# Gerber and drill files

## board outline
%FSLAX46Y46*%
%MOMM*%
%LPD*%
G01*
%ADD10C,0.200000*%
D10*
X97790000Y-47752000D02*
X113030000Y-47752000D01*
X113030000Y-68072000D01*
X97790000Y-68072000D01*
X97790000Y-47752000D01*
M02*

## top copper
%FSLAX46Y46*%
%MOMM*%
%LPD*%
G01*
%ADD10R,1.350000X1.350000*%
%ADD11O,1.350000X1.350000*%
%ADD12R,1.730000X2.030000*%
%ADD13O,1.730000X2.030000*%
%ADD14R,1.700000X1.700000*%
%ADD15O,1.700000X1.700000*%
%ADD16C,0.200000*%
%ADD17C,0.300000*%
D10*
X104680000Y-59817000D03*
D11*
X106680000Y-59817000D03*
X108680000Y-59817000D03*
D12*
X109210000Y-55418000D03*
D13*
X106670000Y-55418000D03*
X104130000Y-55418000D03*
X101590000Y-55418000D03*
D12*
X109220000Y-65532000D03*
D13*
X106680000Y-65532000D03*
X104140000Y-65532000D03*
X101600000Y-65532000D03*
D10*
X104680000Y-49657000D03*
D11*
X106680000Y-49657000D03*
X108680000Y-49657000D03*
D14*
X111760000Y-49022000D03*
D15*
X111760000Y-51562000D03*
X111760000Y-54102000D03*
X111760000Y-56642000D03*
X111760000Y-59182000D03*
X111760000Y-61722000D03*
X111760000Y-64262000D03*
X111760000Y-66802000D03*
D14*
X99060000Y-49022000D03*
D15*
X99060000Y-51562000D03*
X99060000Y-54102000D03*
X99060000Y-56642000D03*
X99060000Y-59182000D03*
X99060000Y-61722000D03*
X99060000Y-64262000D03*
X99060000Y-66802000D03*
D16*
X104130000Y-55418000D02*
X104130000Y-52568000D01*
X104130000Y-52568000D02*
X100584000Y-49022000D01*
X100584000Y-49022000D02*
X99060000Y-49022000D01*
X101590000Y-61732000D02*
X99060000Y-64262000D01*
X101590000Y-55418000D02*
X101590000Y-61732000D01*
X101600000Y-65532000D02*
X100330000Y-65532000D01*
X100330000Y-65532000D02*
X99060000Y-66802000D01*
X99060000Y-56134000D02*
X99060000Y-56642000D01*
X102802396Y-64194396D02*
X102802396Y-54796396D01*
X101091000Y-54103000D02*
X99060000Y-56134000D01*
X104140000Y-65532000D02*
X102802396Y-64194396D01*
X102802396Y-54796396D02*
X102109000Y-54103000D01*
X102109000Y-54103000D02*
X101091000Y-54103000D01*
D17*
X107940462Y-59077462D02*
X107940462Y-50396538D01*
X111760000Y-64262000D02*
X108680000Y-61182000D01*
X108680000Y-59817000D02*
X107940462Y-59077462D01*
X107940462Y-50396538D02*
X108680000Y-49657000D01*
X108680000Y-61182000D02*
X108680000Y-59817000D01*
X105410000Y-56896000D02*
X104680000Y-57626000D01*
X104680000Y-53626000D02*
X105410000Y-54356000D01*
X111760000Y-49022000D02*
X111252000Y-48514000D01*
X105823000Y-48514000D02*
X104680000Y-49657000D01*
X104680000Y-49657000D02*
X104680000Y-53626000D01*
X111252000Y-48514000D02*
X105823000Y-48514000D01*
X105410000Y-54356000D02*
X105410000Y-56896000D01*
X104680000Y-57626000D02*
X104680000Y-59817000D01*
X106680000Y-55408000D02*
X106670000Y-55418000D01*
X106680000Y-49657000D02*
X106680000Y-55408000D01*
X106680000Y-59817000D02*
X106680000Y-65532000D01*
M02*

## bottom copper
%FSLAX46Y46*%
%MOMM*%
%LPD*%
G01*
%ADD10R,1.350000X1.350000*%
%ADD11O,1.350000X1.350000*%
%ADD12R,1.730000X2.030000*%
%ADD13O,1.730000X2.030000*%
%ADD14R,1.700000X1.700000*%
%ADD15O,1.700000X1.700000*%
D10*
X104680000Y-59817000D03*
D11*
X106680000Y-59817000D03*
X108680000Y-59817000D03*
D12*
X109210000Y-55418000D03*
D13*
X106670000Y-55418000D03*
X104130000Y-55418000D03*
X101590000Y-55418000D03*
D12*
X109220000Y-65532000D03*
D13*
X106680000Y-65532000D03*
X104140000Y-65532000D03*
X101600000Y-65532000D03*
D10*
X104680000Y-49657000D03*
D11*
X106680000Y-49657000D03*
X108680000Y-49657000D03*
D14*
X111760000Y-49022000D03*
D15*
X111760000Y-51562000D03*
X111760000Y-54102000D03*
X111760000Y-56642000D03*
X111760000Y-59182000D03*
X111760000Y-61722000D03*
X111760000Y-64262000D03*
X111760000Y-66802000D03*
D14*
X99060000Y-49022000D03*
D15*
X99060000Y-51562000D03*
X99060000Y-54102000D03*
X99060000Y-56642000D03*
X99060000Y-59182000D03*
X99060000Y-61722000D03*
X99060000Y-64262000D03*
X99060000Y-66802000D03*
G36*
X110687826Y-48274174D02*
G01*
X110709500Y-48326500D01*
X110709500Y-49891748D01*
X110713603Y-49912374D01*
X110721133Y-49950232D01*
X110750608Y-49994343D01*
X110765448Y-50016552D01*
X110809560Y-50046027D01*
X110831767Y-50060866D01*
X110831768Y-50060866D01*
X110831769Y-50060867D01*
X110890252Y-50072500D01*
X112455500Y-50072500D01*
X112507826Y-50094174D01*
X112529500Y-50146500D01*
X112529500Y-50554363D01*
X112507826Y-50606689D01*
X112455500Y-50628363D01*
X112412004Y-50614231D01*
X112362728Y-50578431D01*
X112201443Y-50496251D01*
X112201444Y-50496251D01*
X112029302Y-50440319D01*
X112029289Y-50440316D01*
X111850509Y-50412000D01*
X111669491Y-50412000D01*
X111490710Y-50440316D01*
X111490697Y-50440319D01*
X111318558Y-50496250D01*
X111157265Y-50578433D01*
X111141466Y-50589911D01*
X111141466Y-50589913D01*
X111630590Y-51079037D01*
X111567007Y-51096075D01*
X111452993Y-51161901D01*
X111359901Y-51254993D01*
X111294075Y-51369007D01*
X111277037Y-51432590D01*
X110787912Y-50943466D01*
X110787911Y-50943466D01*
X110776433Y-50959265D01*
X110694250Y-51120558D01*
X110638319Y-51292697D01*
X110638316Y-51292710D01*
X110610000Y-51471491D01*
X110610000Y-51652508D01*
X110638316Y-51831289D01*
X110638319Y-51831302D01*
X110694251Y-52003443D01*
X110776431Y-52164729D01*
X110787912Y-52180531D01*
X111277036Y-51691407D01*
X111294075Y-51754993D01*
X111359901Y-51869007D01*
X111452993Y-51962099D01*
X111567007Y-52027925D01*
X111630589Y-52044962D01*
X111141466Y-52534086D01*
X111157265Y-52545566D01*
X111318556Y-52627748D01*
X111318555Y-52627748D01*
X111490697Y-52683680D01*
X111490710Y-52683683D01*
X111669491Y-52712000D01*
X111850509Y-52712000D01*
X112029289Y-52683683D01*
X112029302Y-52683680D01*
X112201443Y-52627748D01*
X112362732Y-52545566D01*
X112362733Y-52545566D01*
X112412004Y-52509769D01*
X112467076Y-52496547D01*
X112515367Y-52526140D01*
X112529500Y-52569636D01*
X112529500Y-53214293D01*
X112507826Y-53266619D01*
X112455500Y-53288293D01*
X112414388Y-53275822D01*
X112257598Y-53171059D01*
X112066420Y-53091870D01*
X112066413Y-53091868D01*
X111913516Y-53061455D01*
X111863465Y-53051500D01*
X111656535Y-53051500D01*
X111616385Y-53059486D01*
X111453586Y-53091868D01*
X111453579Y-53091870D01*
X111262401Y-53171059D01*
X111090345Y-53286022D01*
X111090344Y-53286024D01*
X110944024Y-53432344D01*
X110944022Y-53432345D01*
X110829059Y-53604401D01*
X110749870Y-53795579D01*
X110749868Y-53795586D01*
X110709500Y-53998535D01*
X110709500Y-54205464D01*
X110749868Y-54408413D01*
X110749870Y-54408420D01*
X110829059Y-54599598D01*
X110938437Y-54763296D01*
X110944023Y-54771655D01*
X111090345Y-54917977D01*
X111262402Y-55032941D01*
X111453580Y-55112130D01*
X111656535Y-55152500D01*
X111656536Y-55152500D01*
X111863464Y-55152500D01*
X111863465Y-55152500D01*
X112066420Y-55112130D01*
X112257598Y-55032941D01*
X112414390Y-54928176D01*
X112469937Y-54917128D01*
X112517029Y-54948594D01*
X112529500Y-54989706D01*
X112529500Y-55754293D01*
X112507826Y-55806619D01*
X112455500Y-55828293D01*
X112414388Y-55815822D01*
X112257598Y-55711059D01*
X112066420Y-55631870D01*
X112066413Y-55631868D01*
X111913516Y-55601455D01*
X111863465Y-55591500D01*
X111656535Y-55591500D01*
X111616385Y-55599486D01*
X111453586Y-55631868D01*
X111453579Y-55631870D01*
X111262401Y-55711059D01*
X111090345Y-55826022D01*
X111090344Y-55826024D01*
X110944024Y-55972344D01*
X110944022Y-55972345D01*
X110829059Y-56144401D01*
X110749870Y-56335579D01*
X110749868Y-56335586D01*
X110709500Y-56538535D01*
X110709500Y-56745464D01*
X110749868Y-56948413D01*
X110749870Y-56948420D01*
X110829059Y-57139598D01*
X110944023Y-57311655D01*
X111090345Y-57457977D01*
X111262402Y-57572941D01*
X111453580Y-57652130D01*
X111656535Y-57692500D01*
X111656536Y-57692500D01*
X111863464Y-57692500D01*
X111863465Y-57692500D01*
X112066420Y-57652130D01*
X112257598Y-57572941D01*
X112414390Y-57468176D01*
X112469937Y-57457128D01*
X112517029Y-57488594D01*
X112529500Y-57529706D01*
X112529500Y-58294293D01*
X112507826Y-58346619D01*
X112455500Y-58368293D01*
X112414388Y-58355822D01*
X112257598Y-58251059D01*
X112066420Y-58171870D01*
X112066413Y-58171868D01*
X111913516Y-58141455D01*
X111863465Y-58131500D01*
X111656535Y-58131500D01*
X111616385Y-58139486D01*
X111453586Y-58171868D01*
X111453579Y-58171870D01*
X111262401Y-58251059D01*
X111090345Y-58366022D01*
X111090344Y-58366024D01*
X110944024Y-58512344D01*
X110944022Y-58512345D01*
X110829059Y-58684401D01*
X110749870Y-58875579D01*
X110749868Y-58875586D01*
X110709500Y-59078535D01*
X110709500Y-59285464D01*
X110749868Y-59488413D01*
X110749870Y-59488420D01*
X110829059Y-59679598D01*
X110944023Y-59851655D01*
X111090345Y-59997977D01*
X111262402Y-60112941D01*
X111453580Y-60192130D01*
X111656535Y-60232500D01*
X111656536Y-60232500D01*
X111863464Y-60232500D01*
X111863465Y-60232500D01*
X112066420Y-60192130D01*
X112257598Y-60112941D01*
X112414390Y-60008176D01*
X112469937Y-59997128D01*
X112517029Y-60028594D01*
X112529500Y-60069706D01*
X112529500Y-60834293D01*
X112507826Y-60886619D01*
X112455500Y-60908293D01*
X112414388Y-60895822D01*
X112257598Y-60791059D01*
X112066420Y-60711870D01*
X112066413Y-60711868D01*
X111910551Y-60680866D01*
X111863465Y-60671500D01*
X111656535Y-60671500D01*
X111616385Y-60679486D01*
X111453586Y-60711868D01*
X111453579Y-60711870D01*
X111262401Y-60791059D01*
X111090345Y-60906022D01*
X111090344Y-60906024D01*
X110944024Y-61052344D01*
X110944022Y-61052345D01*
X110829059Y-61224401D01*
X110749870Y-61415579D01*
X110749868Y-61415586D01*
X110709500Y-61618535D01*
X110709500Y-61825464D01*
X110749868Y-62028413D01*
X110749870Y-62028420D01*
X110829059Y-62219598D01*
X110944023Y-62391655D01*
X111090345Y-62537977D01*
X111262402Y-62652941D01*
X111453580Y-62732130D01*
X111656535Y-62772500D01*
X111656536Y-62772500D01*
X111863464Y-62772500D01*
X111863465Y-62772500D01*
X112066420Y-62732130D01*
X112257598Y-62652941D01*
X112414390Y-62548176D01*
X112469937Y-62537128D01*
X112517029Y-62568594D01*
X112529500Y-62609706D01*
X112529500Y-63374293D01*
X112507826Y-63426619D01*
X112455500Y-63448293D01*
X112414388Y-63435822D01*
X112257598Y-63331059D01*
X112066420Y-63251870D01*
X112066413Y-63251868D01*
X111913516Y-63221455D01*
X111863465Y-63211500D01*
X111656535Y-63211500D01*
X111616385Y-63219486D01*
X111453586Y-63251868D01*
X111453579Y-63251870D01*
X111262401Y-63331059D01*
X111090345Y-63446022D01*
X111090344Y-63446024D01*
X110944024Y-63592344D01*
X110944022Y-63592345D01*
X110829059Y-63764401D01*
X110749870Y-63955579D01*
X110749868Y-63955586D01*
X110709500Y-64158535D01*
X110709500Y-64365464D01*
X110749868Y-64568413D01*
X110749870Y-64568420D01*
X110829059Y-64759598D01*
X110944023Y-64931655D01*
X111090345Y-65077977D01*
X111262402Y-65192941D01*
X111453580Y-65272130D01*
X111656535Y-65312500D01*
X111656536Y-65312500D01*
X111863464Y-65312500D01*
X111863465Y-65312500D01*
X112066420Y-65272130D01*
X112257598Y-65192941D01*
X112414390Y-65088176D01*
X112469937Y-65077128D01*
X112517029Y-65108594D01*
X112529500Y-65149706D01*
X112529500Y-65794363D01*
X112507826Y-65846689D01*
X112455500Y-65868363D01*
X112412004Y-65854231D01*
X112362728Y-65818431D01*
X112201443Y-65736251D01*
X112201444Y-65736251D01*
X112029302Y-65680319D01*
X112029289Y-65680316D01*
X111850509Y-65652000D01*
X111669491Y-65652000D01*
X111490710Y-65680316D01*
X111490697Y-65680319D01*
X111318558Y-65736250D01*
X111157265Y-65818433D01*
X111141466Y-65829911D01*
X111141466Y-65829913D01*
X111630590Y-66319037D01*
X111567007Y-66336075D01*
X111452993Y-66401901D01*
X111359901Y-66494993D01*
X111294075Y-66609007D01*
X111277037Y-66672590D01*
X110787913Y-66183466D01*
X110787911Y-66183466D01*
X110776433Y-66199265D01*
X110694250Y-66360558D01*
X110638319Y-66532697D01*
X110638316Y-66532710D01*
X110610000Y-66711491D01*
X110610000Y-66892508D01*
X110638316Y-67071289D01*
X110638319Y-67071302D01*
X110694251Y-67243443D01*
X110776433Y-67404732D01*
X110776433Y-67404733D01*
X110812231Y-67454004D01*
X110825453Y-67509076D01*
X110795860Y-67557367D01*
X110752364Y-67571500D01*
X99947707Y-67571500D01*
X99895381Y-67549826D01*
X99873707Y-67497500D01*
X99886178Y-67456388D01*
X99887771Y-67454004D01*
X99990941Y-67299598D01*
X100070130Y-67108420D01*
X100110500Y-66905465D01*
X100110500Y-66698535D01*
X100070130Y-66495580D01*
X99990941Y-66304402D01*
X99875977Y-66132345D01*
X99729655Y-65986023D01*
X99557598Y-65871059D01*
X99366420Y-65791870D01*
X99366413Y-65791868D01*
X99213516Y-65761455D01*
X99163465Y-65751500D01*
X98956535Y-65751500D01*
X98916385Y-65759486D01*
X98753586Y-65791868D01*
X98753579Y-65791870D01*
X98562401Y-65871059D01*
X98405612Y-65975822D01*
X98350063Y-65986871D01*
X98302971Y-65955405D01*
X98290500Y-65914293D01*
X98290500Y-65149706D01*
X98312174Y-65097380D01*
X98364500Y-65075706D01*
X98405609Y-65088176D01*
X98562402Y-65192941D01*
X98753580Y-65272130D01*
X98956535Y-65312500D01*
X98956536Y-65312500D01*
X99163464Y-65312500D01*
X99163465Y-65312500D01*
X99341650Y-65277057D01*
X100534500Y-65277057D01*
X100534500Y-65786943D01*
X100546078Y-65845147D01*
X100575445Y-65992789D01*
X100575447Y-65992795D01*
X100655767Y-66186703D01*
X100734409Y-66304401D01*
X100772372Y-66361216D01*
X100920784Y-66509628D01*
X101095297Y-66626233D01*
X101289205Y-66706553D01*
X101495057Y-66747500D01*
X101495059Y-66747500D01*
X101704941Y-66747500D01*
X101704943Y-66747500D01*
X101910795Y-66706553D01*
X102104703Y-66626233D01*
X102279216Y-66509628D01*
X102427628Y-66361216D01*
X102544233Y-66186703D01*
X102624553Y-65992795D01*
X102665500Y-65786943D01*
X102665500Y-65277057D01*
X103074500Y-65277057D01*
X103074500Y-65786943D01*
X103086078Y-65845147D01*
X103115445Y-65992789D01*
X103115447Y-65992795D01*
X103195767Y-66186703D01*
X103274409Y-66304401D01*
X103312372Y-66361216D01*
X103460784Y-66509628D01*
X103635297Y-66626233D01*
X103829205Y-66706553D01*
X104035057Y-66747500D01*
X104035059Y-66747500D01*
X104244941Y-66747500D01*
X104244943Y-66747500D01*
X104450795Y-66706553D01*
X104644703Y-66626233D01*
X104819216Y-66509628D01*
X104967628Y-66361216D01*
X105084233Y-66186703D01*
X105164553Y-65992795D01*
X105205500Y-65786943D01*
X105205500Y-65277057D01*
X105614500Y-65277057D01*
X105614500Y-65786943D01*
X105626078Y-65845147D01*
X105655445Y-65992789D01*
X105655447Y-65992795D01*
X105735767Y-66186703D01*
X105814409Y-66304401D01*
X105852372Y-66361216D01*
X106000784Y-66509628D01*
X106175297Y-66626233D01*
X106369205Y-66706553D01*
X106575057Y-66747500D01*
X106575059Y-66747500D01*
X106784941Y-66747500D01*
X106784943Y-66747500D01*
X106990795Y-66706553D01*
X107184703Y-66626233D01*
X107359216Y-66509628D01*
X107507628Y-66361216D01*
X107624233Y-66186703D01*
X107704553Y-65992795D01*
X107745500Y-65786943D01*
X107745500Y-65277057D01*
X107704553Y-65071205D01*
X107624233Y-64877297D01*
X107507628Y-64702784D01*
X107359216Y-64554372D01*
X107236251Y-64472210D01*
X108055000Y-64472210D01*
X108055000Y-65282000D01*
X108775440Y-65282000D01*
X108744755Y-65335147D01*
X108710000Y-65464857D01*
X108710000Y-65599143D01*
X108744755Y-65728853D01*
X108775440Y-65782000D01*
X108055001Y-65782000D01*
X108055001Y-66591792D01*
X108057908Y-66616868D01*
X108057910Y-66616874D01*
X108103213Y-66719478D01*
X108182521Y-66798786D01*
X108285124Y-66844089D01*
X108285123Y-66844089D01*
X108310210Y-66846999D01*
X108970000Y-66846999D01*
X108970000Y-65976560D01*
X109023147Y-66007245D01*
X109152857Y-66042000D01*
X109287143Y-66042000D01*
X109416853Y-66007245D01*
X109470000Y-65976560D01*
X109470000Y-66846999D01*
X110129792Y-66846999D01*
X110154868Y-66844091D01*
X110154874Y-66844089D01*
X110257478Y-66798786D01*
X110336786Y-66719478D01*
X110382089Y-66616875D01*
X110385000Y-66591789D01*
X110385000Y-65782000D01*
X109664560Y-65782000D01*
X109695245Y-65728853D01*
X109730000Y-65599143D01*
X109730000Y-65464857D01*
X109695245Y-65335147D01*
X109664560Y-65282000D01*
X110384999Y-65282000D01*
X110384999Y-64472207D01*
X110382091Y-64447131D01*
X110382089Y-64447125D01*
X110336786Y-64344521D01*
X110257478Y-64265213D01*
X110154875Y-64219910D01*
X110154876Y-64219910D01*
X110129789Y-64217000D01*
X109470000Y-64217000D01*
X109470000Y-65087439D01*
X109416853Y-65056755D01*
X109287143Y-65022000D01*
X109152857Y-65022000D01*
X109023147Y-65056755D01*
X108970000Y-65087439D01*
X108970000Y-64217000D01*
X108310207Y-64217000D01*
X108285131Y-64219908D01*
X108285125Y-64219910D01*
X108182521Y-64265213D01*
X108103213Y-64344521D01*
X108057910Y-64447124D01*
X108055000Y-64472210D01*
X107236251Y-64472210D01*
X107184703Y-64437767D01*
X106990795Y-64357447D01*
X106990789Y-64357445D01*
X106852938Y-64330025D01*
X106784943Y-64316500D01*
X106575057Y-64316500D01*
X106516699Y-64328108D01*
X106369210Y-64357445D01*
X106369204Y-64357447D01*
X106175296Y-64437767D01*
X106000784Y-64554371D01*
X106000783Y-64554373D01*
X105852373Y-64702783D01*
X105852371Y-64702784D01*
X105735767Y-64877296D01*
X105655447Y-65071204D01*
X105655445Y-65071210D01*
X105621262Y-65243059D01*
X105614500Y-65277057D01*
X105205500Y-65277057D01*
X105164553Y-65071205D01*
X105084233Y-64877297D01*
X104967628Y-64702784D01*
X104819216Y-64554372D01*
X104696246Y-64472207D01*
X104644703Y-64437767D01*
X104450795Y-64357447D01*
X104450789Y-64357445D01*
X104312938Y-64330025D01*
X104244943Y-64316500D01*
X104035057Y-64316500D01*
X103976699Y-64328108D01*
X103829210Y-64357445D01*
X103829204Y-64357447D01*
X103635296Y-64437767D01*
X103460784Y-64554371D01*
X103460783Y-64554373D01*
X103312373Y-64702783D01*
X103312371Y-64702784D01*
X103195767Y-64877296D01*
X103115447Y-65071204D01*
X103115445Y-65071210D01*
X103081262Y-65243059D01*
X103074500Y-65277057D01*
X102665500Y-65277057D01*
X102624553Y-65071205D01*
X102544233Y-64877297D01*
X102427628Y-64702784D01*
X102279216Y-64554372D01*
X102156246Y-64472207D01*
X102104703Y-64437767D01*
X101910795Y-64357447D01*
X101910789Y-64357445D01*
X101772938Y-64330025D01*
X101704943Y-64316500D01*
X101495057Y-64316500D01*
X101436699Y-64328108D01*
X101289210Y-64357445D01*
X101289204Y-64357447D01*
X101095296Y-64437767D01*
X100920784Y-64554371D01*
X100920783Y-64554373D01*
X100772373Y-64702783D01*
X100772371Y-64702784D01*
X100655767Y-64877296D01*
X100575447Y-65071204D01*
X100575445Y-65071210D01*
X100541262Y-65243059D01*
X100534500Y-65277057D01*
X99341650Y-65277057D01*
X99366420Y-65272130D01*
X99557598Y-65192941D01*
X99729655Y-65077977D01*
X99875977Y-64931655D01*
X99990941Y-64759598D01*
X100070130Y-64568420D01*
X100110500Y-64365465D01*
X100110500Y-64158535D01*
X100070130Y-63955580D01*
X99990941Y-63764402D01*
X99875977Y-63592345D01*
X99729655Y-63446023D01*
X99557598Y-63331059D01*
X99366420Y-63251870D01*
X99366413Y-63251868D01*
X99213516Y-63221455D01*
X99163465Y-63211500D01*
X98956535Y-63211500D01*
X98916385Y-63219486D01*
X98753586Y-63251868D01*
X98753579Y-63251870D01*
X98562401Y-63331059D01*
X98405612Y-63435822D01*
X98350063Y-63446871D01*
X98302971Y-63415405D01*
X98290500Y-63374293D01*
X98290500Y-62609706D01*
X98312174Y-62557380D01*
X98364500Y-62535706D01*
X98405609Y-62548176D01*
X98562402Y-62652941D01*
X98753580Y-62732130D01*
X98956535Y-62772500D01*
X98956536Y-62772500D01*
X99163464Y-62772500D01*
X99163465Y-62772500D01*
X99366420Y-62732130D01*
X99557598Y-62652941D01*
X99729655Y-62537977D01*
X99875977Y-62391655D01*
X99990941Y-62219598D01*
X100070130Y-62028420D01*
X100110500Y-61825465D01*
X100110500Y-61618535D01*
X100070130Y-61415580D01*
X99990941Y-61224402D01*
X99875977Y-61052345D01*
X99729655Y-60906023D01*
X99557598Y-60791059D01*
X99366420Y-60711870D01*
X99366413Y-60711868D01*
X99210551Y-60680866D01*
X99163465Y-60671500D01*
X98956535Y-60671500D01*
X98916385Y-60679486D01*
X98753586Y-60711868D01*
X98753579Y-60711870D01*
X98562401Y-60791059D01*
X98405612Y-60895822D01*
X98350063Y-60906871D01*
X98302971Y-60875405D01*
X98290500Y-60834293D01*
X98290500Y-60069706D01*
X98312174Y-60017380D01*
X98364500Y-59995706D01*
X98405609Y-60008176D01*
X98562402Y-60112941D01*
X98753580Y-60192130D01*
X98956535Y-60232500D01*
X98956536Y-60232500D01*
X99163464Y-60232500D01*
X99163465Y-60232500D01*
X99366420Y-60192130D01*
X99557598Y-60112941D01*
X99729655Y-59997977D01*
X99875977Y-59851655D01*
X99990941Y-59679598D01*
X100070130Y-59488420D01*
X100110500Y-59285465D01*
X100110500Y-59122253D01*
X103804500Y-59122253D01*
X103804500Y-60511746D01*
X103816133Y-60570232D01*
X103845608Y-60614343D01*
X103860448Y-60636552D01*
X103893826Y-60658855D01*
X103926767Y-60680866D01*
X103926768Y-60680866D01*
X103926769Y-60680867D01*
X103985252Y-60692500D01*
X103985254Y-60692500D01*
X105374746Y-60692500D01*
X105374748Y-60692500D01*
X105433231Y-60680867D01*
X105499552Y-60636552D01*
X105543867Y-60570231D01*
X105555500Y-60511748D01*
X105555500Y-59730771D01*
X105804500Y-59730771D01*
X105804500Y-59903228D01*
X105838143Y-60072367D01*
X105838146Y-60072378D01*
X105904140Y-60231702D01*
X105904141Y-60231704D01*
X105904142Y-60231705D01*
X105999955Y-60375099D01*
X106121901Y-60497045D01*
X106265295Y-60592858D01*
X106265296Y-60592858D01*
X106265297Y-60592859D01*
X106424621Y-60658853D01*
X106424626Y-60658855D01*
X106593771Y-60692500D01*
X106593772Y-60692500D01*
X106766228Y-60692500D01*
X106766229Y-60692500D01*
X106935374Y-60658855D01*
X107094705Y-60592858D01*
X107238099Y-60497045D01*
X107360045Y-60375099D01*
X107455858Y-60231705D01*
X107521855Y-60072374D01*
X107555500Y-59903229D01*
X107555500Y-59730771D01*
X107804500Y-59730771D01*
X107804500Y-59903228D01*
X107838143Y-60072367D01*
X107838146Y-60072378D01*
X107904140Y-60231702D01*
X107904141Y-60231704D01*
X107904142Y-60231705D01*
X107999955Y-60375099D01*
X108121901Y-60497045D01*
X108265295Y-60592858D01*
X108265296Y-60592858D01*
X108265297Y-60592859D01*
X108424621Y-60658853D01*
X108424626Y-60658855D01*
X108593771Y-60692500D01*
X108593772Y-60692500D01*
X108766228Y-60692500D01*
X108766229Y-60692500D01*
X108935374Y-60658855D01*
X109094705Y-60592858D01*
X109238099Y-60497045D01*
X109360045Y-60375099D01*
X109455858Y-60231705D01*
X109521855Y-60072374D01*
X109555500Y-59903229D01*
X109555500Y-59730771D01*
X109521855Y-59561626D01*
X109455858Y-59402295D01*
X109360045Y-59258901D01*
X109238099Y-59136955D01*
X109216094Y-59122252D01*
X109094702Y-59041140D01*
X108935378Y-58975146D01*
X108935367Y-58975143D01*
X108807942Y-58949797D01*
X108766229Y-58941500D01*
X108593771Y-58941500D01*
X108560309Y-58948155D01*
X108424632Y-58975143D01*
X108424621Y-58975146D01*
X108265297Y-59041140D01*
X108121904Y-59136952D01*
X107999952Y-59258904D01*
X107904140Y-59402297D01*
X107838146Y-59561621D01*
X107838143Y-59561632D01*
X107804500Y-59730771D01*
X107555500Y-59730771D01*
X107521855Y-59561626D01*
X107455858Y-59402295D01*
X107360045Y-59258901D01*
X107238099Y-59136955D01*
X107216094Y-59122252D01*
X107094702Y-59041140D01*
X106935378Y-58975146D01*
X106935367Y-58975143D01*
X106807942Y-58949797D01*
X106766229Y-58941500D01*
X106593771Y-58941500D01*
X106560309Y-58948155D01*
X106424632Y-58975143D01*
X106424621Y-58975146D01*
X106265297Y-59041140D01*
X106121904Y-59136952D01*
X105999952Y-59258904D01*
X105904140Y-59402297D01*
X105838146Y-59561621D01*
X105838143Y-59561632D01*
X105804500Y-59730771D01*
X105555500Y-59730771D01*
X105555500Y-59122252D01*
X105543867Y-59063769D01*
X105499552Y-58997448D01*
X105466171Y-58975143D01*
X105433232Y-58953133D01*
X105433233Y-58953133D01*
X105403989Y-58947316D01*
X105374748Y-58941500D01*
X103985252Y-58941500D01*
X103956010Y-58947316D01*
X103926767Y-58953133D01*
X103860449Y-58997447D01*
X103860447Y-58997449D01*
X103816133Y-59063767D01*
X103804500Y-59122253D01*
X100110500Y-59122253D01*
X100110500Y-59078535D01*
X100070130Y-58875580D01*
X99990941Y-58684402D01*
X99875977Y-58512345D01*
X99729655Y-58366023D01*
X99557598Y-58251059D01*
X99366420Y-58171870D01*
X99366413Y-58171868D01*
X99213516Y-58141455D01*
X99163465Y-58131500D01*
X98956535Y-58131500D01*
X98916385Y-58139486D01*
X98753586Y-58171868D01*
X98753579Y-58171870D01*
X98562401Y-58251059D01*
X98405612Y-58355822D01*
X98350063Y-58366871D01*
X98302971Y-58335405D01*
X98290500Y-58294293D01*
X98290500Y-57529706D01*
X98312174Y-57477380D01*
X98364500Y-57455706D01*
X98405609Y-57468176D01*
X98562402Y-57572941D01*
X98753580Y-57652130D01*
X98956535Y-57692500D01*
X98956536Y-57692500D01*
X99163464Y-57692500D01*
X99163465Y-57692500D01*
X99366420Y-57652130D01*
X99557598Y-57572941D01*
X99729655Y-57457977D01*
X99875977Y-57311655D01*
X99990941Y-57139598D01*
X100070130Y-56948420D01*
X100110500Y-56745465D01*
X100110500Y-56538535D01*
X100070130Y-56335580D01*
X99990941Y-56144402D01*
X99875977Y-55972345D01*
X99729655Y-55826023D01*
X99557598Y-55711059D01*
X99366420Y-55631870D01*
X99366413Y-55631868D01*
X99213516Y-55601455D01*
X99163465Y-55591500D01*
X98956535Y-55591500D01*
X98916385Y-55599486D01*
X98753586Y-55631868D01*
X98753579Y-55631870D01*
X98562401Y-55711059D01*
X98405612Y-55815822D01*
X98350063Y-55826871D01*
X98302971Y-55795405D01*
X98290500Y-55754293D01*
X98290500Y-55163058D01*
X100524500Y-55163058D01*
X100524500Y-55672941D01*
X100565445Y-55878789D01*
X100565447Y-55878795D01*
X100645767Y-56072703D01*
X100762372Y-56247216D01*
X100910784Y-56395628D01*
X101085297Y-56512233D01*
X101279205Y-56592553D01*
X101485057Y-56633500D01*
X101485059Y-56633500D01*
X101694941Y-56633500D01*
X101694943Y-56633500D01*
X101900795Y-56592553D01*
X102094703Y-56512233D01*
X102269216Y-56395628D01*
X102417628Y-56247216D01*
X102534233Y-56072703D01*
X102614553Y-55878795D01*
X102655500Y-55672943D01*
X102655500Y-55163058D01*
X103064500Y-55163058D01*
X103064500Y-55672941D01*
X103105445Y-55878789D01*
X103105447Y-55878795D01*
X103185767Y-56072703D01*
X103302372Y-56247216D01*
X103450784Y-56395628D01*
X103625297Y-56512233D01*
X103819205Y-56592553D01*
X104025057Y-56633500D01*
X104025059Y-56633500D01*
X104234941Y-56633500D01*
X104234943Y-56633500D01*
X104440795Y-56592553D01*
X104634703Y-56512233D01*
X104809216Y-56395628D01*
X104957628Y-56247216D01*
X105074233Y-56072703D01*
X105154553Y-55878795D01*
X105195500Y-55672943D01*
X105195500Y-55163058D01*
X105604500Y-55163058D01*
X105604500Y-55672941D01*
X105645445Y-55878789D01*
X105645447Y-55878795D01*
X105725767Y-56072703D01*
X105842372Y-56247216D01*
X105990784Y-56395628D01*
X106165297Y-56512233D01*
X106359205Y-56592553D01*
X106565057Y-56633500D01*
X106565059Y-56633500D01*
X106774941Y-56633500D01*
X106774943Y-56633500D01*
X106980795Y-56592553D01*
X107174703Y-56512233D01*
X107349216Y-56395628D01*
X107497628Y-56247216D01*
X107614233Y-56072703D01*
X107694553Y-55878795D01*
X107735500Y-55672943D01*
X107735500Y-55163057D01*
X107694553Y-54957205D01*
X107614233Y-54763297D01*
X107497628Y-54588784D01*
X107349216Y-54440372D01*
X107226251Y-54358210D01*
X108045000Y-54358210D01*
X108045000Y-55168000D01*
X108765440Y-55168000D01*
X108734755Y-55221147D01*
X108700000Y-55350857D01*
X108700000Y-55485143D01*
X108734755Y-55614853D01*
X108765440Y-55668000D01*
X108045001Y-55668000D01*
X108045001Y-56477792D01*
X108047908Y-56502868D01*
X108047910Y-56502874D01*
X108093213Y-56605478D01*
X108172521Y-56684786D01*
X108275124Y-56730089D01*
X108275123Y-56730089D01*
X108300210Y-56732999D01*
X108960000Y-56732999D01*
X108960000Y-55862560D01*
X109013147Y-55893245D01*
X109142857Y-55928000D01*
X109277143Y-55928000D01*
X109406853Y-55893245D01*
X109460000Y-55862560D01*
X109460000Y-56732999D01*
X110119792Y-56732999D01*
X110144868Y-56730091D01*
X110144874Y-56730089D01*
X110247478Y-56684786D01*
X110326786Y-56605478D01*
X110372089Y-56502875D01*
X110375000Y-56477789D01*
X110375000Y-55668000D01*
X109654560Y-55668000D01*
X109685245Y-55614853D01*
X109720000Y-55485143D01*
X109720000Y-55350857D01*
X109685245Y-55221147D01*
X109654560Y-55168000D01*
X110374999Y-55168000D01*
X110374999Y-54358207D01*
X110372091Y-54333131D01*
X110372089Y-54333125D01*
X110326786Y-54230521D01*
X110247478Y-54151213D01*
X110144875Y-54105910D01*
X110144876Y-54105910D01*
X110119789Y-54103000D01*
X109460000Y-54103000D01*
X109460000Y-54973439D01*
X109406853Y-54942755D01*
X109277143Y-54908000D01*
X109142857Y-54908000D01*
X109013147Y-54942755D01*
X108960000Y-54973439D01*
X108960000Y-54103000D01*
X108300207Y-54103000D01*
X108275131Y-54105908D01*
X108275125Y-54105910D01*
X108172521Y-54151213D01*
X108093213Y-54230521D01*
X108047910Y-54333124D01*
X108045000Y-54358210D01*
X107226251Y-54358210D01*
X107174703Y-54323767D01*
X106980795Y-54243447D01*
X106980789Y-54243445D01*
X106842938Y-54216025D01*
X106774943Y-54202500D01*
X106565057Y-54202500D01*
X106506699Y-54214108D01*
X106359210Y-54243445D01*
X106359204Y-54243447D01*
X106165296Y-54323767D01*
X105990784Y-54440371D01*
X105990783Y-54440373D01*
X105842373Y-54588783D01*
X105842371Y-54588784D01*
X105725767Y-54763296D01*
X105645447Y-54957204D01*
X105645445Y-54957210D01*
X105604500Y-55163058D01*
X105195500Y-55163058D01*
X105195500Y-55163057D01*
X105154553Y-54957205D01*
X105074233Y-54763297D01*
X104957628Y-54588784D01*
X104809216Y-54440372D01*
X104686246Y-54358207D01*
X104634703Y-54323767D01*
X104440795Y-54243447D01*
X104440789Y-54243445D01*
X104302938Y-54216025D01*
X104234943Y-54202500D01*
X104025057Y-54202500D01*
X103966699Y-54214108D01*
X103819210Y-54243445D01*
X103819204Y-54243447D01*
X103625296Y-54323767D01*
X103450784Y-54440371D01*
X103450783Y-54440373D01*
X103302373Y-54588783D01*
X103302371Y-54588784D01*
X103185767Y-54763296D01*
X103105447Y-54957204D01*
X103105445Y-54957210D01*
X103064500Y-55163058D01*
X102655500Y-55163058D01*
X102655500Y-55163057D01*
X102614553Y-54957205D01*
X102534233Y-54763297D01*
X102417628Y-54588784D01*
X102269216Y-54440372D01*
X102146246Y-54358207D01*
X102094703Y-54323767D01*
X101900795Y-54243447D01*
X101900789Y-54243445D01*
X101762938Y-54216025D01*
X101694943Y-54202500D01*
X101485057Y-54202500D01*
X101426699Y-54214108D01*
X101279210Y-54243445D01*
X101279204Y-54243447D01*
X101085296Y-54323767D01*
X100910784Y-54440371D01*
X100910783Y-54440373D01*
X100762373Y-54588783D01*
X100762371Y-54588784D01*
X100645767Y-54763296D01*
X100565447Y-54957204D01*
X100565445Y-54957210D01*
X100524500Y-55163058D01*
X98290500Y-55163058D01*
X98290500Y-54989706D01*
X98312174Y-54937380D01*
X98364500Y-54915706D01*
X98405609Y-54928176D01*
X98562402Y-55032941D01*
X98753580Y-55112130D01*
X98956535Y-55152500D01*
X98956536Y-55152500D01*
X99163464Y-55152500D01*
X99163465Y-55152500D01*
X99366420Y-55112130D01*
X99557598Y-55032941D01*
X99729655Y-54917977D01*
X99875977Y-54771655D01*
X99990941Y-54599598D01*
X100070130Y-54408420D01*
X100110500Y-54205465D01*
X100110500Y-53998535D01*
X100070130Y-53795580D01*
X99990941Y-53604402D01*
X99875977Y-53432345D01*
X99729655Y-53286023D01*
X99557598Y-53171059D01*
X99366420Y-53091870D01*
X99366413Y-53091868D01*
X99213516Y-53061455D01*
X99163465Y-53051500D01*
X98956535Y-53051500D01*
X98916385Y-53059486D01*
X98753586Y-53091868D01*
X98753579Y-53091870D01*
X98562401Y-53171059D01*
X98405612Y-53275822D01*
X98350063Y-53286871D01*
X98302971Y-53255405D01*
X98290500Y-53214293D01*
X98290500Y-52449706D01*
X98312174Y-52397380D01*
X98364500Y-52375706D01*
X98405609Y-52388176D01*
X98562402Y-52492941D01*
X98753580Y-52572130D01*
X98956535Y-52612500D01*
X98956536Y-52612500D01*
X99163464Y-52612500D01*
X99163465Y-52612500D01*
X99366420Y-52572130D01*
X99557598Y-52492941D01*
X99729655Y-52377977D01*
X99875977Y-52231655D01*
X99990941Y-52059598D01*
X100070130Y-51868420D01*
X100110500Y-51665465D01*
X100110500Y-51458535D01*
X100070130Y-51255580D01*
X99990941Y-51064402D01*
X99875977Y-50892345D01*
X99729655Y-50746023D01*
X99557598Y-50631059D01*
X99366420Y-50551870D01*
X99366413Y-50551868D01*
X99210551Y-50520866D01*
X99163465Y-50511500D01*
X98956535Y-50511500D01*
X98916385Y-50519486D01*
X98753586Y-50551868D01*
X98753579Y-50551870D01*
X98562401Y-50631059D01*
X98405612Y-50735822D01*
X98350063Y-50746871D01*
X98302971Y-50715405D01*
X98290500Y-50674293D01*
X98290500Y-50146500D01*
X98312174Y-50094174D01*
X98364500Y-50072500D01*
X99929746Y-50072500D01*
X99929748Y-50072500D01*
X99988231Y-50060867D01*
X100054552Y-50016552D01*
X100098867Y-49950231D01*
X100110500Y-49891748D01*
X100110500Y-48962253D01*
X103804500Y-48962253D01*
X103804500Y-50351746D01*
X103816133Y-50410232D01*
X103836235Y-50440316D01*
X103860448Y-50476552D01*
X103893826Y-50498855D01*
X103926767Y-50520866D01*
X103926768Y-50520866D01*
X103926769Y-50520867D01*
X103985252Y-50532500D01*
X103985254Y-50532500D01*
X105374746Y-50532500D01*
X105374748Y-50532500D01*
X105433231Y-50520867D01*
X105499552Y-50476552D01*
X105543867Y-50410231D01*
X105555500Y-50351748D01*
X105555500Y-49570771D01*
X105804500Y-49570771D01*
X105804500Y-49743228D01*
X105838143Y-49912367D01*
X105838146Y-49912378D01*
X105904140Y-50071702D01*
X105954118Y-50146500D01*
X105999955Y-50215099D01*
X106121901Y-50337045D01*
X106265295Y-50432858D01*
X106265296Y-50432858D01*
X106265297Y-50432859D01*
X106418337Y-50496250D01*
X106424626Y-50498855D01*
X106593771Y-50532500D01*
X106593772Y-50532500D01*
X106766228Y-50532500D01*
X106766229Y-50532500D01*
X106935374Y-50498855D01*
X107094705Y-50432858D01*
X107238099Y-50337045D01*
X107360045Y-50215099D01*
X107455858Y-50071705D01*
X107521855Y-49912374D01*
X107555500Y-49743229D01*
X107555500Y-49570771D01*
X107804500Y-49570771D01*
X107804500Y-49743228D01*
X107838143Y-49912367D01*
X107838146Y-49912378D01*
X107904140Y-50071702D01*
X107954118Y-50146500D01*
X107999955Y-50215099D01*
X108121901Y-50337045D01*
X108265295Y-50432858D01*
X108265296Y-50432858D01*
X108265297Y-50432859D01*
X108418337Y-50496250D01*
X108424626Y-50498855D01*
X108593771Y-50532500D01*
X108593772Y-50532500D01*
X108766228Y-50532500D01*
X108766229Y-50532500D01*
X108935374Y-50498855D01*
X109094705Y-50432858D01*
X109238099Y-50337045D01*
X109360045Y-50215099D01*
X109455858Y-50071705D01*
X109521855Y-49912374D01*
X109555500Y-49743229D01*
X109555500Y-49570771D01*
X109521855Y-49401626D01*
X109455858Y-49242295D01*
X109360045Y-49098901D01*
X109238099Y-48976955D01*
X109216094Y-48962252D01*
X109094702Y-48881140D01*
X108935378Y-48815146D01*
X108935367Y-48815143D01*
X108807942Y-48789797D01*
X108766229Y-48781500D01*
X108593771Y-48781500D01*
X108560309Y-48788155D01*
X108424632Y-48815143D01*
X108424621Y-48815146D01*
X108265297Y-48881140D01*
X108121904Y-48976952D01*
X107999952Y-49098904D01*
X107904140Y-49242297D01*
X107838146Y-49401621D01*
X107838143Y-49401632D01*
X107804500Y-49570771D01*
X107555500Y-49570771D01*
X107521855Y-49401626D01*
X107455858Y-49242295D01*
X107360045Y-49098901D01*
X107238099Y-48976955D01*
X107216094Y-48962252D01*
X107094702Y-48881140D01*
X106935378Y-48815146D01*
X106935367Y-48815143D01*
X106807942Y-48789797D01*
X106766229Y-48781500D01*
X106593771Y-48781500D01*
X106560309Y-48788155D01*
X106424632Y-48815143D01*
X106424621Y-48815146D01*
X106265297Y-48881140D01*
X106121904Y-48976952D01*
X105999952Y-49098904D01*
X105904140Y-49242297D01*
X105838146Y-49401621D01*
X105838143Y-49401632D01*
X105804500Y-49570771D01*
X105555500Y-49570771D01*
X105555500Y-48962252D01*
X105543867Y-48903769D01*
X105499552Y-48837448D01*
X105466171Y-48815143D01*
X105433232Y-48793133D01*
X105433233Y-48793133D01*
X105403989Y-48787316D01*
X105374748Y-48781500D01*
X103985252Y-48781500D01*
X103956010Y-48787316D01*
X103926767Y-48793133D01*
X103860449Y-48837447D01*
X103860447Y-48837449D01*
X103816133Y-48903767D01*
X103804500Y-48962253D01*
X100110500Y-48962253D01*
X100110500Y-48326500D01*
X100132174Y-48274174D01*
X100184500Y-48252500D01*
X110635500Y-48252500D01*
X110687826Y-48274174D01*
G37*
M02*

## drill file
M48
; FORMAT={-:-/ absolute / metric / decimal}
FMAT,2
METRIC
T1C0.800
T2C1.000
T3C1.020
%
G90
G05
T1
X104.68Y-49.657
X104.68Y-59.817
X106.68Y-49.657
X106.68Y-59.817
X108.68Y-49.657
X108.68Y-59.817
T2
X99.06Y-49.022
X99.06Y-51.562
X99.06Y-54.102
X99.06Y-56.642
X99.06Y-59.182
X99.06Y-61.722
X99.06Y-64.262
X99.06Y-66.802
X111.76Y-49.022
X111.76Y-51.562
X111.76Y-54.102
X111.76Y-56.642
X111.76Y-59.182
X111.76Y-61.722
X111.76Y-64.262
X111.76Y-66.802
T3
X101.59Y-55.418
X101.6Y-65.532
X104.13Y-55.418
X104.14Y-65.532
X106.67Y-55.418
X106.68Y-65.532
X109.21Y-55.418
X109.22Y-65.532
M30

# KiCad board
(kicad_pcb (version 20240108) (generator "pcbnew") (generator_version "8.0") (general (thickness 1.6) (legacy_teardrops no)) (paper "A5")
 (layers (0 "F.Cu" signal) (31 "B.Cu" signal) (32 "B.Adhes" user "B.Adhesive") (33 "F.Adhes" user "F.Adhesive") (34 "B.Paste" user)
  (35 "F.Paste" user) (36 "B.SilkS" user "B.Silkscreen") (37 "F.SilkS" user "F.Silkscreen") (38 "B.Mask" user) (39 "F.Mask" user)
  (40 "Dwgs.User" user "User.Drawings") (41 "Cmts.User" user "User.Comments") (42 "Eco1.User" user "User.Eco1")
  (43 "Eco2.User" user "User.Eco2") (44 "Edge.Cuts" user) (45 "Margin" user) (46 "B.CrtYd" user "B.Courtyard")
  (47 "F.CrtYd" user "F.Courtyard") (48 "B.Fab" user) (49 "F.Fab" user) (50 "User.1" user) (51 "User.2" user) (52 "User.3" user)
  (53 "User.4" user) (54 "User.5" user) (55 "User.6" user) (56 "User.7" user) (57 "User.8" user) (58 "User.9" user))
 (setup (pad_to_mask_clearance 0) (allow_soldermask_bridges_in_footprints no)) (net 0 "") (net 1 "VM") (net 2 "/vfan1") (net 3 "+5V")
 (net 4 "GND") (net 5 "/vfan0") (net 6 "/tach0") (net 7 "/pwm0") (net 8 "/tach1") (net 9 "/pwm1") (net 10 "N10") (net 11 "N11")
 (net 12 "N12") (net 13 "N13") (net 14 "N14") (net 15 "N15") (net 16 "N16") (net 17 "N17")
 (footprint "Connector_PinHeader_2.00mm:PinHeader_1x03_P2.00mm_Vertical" (layer "F.Cu") (at 104.68 59.817 90)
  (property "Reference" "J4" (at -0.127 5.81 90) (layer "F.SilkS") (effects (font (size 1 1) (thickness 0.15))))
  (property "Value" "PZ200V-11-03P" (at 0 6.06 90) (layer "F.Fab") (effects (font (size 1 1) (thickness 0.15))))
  (pad "1" thru_hole rect (at 0 0 90) (size 1.35 1.35) (drill 0.8) (layers "*.Cu" "*.Mask") (remove_unused_layers no) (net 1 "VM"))
  (pad "2" thru_hole oval (at 0 2 90) (size 1.35 1.35) (drill 0.8) (layers "*.Cu" "*.Mask") (remove_unused_layers no) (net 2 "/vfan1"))
  (pad "3" thru_hole oval (at 0 4 90) (size 1.35 1.35) (drill 0.8) (layers "*.Cu" "*.Mask") (remove_unused_layers no) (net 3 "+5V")))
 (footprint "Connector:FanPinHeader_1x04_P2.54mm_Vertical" (layer "F.Cu") (at 109.21 55.418 180)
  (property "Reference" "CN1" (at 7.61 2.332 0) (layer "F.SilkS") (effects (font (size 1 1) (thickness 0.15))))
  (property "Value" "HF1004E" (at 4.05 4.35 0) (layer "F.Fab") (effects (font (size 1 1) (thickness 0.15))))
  (pad "1" thru_hole rect (at 0 0 270) (size 2.03 1.73) (drill 1.02) (layers "*.Cu" "*.Mask") (remove_unused_layers no) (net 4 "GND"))
  (pad "2" thru_hole oval (at 2.54 0 270) (size 2.03 1.73) (drill 1.02) (layers "*.Cu" "*.Mask") (remove_unused_layers no) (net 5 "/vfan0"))
  (pad "3" thru_hole oval (at 5.08 0 270) (size 2.03 1.73) (drill 1.02) (layers "*.Cu" "*.Mask") (remove_unused_layers no) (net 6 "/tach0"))
  (pad "4" thru_hole oval (at 7.62 0 270) (size 2.03 1.73) (drill 1.02) (layers "*.Cu" "*.Mask") (remove_unused_layers no) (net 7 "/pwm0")
   (thermal_bridge_angle 45)))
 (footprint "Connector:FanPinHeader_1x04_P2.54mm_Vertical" (layer "F.Cu") (at 109.22 65.532 180)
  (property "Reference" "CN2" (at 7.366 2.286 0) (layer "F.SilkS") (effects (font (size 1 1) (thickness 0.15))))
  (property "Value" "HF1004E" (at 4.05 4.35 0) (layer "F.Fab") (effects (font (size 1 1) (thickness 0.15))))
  (pad "1" thru_hole rect (at 0 0 270) (size 2.03 1.73) (drill 1.02) (layers "*.Cu" "*.Mask") (remove_unused_layers no) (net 4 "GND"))
  (pad "2" thru_hole oval (at 2.54 0 270) (size 2.03 1.73) (drill 1.02) (layers "*.Cu" "*.Mask") (remove_unused_layers no) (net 2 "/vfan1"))
  (pad "3" thru_hole oval (at 5.08 0 270) (size 2.03 1.73) (drill 1.02) (layers "*.Cu" "*.Mask") (remove_unused_layers no) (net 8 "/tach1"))
  (pad "4" thru_hole oval (at 7.62 0 270) (size 2.03 1.73) (drill 1.02) (layers "*.Cu" "*.Mask") (remove_unused_layers no) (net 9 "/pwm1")
   (thermal_bridge_angle 45)))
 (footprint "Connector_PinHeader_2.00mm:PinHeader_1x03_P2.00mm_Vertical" (layer "F.Cu") (at 104.68 49.657 90)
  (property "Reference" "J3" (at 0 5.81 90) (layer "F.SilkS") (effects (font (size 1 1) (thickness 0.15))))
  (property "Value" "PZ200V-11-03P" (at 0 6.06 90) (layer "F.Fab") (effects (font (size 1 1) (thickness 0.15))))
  (pad "1" thru_hole rect (at 0 0 90) (size 1.35 1.35) (drill 0.8) (layers "*.Cu" "*.Mask") (remove_unused_layers no) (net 1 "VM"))
  (pad "2" thru_hole oval (at 0 2 90) (size 1.35 1.35) (drill 0.8) (layers "*.Cu" "*.Mask") (remove_unused_layers no) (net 5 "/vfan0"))
  (pad "3" thru_hole oval (at 0 4 90) (size 1.35 1.35) (drill 0.8) (layers "*.Cu" "*.Mask") (remove_unused_layers no) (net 3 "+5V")))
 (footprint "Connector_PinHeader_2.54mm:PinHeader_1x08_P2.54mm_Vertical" (layer "B.Cu") (at 111.76 49.022 180)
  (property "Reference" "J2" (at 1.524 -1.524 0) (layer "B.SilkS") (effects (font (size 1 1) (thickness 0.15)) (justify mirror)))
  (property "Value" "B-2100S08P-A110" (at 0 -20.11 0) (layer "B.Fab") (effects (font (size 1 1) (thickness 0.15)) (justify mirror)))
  (pad "1" thru_hole rect (at 0 0 180) (size 1.7 1.7) (drill 1) (layers "*.Cu" "*.Mask") (remove_unused_layers no) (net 1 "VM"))
  (pad "2" thru_hole oval (at 0 -2.54 180) (size 1.7 1.7) (drill 1) (layers "*.Cu" "*.Mask") (remove_unused_layers no) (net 4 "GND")
   (thermal_bridge_angle 45))
  (pad "3" thru_hole oval (at 0 -5.08 180) (size 1.7 1.7) (drill 1) (layers "*.Cu" "*.Mask") (remove_unused_layers no) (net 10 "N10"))
  (pad "4" thru_hole oval (at 0 -7.62 180) (size 1.7 1.7) (drill 1) (layers "*.Cu" "*.Mask") (remove_unused_layers no) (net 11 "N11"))
  (pad "5" thru_hole oval (at 0 -10.16 180) (size 1.7 1.7) (drill 1) (layers "*.Cu" "*.Mask") (remove_unused_layers no) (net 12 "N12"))
  (pad "6" thru_hole oval (at 0 -12.7 180) (size 1.7 1.7) (drill 1) (layers "*.Cu" "*.Mask") (remove_unused_layers no) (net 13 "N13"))
  (pad "7" thru_hole oval (at 0 -15.24 180) (size 1.7 1.7) (drill 1) (layers "*.Cu" "*.Mask") (remove_unused_layers no) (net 3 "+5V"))
  (pad "8" thru_hole oval (at 0 -17.78 180) (size 1.7 1.7) (drill 1) (layers "*.Cu" "*.Mask") (remove_unused_layers no) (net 4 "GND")
   (thermal_bridge_angle 45)))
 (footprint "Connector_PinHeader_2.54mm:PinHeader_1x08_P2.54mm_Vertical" (layer "B.Cu") (at 99.06 49.022 180)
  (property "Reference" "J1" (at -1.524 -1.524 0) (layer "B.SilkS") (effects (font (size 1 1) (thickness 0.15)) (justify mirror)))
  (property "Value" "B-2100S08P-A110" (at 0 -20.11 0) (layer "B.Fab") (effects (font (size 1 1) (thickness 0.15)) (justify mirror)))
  (pad "1" thru_hole rect (at 0 0 180) (size 1.7 1.7) (drill 1) (layers "*.Cu" "*.Mask") (remove_unused_layers no) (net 6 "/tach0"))
  (pad "2" thru_hole oval (at 0 -2.54 180) (size 1.7 1.7) (drill 1) (layers "*.Cu" "*.Mask") (remove_unused_layers no) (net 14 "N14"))
  (pad "3" thru_hole oval (at 0 -5.08 180) (size 1.7 1.7) (drill 1) (layers "*.Cu" "*.Mask") (remove_unused_layers no) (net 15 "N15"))
  (pad "4" thru_hole oval (at 0 -7.62 180) (size 1.7 1.7) (drill 1) (layers "*.Cu" "*.Mask") (remove_unused_layers no) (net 8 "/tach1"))
  (pad "5" thru_hole oval (at 0 -10.16 180) (size 1.7 1.7) (drill 1) (layers "*.Cu" "*.Mask") (remove_unused_layers no) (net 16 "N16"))
  (pad "6" thru_hole oval (at 0 -12.7 180) (size 1.7 1.7) (drill 1) (layers "*.Cu" "*.Mask") (remove_unused_layers no) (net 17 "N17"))
  (pad "7" thru_hole oval (at 0 -15.24 180) (size 1.7 1.7) (drill 1) (layers "*.Cu" "*.Mask") (remove_unused_layers no) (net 7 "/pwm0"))
  (pad "8" thru_hole oval (at 0 -17.78 180) (size 1.7 1.7) (drill 1) (layers "*.Cu" "*.Mask") (remove_unused_layers no) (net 9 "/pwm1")))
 (gr_rect (start 97.79 47.752) (end 113.03 68.072) (stroke (width 0.2) (type default)) (fill none) (layer "Edge.Cuts"))
 (segment (start 104.13 55.418) (end 104.13 52.568) (width 0.2) (layer "F.Cu") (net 6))
 (segment (start 104.13 52.568) (end 100.584 49.022) (width 0.2) (layer "F.Cu") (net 6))
 (segment (start 100.584 49.022) (end 99.06 49.022) (width 0.2) (layer "F.Cu") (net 6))
 (segment (start 101.59 61.732) (end 99.06 64.262) (width 0.2) (layer "F.Cu") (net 7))
 (segment (start 101.59 55.418) (end 101.59 61.732) (width 0.2) (layer "F.Cu") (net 7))
 (segment (start 101.6 65.532) (end 100.33 65.532) (width 0.2) (layer "F.Cu") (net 9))
 (segment (start 100.33 65.532) (end 99.06 66.802) (width 0.2) (layer "F.Cu") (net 9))
 (segment (start 99.06 56.134) (end 99.06 56.642) (width 0.2) (layer "F.Cu") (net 8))
 (segment (start 102.802396 64.194396) (end 102.802396 54.796396) (width 0.2) (layer "F.Cu") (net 8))
 (segment (start 101.091 54.103) (end 99.06 56.134) (width 0.2) (layer "F.Cu") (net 8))
 (segment (start 104.14 65.532) (end 102.802396 64.194396) (width 0.2) (layer "F.Cu") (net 8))
 (segment (start 102.802396 54.796396) (end 102.109 54.103) (width 0.2) (layer "F.Cu") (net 8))
 (segment (start 102.109 54.103) (end 101.091 54.103) (width 0.2) (layer "F.Cu") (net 8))
 (segment (start 107.940462 59.077462) (end 107.940462 50.396538) (width 0.3) (layer "F.Cu") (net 3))
 (segment (start 111.76 64.262) (end 108.68 61.182) (width 0.3) (layer "F.Cu") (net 3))
 (segment (start 108.68 59.817) (end 107.940462 59.077462) (width 0.3) (layer "F.Cu") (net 3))
 (segment (start 107.940462 50.396538) (end 108.68 49.657) (width 0.3) (layer "F.Cu") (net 3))
 (segment (start 108.68 61.182) (end 108.68 59.817) (width 0.3) (layer "F.Cu") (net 3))
 (segment (start 105.41 56.896) (end 104.68 57.626) (width 0.3) (layer "F.Cu") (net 1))
 (segment (start 104.68 53.626) (end 105.41 54.356) (width 0.3) (layer "F.Cu") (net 1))
 (segment (start 111.76 49.022) (end 111.252 48.514) (width 0.3) (layer "F.Cu") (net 1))
 (segment (start 105.823 48.514) (end 104.68 49.657) (width 0.3) (layer "F.Cu") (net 1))
 (segment (start 104.68 49.657) (end 104.68 53.626) (width 0.3) (layer "F.Cu") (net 1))
 (segment (start 111.252 48.514) (end 105.823 48.514) (width 0.3) (layer "F.Cu") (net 1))
 (segment (start 105.41 54.356) (end 105.41 56.896) (width 0.3) (layer "F.Cu") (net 1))
 (segment (start 104.68 57.626) (end 104.68 59.817) (width 0.3) (layer "F.Cu") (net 1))
 (segment (start 106.68 55.408) (end 106.67 55.418) (width 0.3) (layer "F.Cu") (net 5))
 (segment (start 106.68 49.657) (end 106.68 55.408) (width 0.3) (layer "F.Cu") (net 5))
 (segment (start 106.68 59.817) (end 106.68 65.532) (width 0.3) (layer "F.Cu") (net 2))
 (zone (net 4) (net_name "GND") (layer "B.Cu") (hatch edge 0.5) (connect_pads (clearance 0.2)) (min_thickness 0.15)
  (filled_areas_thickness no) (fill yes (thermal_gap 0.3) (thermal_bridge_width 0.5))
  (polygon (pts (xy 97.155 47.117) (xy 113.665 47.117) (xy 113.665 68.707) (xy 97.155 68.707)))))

